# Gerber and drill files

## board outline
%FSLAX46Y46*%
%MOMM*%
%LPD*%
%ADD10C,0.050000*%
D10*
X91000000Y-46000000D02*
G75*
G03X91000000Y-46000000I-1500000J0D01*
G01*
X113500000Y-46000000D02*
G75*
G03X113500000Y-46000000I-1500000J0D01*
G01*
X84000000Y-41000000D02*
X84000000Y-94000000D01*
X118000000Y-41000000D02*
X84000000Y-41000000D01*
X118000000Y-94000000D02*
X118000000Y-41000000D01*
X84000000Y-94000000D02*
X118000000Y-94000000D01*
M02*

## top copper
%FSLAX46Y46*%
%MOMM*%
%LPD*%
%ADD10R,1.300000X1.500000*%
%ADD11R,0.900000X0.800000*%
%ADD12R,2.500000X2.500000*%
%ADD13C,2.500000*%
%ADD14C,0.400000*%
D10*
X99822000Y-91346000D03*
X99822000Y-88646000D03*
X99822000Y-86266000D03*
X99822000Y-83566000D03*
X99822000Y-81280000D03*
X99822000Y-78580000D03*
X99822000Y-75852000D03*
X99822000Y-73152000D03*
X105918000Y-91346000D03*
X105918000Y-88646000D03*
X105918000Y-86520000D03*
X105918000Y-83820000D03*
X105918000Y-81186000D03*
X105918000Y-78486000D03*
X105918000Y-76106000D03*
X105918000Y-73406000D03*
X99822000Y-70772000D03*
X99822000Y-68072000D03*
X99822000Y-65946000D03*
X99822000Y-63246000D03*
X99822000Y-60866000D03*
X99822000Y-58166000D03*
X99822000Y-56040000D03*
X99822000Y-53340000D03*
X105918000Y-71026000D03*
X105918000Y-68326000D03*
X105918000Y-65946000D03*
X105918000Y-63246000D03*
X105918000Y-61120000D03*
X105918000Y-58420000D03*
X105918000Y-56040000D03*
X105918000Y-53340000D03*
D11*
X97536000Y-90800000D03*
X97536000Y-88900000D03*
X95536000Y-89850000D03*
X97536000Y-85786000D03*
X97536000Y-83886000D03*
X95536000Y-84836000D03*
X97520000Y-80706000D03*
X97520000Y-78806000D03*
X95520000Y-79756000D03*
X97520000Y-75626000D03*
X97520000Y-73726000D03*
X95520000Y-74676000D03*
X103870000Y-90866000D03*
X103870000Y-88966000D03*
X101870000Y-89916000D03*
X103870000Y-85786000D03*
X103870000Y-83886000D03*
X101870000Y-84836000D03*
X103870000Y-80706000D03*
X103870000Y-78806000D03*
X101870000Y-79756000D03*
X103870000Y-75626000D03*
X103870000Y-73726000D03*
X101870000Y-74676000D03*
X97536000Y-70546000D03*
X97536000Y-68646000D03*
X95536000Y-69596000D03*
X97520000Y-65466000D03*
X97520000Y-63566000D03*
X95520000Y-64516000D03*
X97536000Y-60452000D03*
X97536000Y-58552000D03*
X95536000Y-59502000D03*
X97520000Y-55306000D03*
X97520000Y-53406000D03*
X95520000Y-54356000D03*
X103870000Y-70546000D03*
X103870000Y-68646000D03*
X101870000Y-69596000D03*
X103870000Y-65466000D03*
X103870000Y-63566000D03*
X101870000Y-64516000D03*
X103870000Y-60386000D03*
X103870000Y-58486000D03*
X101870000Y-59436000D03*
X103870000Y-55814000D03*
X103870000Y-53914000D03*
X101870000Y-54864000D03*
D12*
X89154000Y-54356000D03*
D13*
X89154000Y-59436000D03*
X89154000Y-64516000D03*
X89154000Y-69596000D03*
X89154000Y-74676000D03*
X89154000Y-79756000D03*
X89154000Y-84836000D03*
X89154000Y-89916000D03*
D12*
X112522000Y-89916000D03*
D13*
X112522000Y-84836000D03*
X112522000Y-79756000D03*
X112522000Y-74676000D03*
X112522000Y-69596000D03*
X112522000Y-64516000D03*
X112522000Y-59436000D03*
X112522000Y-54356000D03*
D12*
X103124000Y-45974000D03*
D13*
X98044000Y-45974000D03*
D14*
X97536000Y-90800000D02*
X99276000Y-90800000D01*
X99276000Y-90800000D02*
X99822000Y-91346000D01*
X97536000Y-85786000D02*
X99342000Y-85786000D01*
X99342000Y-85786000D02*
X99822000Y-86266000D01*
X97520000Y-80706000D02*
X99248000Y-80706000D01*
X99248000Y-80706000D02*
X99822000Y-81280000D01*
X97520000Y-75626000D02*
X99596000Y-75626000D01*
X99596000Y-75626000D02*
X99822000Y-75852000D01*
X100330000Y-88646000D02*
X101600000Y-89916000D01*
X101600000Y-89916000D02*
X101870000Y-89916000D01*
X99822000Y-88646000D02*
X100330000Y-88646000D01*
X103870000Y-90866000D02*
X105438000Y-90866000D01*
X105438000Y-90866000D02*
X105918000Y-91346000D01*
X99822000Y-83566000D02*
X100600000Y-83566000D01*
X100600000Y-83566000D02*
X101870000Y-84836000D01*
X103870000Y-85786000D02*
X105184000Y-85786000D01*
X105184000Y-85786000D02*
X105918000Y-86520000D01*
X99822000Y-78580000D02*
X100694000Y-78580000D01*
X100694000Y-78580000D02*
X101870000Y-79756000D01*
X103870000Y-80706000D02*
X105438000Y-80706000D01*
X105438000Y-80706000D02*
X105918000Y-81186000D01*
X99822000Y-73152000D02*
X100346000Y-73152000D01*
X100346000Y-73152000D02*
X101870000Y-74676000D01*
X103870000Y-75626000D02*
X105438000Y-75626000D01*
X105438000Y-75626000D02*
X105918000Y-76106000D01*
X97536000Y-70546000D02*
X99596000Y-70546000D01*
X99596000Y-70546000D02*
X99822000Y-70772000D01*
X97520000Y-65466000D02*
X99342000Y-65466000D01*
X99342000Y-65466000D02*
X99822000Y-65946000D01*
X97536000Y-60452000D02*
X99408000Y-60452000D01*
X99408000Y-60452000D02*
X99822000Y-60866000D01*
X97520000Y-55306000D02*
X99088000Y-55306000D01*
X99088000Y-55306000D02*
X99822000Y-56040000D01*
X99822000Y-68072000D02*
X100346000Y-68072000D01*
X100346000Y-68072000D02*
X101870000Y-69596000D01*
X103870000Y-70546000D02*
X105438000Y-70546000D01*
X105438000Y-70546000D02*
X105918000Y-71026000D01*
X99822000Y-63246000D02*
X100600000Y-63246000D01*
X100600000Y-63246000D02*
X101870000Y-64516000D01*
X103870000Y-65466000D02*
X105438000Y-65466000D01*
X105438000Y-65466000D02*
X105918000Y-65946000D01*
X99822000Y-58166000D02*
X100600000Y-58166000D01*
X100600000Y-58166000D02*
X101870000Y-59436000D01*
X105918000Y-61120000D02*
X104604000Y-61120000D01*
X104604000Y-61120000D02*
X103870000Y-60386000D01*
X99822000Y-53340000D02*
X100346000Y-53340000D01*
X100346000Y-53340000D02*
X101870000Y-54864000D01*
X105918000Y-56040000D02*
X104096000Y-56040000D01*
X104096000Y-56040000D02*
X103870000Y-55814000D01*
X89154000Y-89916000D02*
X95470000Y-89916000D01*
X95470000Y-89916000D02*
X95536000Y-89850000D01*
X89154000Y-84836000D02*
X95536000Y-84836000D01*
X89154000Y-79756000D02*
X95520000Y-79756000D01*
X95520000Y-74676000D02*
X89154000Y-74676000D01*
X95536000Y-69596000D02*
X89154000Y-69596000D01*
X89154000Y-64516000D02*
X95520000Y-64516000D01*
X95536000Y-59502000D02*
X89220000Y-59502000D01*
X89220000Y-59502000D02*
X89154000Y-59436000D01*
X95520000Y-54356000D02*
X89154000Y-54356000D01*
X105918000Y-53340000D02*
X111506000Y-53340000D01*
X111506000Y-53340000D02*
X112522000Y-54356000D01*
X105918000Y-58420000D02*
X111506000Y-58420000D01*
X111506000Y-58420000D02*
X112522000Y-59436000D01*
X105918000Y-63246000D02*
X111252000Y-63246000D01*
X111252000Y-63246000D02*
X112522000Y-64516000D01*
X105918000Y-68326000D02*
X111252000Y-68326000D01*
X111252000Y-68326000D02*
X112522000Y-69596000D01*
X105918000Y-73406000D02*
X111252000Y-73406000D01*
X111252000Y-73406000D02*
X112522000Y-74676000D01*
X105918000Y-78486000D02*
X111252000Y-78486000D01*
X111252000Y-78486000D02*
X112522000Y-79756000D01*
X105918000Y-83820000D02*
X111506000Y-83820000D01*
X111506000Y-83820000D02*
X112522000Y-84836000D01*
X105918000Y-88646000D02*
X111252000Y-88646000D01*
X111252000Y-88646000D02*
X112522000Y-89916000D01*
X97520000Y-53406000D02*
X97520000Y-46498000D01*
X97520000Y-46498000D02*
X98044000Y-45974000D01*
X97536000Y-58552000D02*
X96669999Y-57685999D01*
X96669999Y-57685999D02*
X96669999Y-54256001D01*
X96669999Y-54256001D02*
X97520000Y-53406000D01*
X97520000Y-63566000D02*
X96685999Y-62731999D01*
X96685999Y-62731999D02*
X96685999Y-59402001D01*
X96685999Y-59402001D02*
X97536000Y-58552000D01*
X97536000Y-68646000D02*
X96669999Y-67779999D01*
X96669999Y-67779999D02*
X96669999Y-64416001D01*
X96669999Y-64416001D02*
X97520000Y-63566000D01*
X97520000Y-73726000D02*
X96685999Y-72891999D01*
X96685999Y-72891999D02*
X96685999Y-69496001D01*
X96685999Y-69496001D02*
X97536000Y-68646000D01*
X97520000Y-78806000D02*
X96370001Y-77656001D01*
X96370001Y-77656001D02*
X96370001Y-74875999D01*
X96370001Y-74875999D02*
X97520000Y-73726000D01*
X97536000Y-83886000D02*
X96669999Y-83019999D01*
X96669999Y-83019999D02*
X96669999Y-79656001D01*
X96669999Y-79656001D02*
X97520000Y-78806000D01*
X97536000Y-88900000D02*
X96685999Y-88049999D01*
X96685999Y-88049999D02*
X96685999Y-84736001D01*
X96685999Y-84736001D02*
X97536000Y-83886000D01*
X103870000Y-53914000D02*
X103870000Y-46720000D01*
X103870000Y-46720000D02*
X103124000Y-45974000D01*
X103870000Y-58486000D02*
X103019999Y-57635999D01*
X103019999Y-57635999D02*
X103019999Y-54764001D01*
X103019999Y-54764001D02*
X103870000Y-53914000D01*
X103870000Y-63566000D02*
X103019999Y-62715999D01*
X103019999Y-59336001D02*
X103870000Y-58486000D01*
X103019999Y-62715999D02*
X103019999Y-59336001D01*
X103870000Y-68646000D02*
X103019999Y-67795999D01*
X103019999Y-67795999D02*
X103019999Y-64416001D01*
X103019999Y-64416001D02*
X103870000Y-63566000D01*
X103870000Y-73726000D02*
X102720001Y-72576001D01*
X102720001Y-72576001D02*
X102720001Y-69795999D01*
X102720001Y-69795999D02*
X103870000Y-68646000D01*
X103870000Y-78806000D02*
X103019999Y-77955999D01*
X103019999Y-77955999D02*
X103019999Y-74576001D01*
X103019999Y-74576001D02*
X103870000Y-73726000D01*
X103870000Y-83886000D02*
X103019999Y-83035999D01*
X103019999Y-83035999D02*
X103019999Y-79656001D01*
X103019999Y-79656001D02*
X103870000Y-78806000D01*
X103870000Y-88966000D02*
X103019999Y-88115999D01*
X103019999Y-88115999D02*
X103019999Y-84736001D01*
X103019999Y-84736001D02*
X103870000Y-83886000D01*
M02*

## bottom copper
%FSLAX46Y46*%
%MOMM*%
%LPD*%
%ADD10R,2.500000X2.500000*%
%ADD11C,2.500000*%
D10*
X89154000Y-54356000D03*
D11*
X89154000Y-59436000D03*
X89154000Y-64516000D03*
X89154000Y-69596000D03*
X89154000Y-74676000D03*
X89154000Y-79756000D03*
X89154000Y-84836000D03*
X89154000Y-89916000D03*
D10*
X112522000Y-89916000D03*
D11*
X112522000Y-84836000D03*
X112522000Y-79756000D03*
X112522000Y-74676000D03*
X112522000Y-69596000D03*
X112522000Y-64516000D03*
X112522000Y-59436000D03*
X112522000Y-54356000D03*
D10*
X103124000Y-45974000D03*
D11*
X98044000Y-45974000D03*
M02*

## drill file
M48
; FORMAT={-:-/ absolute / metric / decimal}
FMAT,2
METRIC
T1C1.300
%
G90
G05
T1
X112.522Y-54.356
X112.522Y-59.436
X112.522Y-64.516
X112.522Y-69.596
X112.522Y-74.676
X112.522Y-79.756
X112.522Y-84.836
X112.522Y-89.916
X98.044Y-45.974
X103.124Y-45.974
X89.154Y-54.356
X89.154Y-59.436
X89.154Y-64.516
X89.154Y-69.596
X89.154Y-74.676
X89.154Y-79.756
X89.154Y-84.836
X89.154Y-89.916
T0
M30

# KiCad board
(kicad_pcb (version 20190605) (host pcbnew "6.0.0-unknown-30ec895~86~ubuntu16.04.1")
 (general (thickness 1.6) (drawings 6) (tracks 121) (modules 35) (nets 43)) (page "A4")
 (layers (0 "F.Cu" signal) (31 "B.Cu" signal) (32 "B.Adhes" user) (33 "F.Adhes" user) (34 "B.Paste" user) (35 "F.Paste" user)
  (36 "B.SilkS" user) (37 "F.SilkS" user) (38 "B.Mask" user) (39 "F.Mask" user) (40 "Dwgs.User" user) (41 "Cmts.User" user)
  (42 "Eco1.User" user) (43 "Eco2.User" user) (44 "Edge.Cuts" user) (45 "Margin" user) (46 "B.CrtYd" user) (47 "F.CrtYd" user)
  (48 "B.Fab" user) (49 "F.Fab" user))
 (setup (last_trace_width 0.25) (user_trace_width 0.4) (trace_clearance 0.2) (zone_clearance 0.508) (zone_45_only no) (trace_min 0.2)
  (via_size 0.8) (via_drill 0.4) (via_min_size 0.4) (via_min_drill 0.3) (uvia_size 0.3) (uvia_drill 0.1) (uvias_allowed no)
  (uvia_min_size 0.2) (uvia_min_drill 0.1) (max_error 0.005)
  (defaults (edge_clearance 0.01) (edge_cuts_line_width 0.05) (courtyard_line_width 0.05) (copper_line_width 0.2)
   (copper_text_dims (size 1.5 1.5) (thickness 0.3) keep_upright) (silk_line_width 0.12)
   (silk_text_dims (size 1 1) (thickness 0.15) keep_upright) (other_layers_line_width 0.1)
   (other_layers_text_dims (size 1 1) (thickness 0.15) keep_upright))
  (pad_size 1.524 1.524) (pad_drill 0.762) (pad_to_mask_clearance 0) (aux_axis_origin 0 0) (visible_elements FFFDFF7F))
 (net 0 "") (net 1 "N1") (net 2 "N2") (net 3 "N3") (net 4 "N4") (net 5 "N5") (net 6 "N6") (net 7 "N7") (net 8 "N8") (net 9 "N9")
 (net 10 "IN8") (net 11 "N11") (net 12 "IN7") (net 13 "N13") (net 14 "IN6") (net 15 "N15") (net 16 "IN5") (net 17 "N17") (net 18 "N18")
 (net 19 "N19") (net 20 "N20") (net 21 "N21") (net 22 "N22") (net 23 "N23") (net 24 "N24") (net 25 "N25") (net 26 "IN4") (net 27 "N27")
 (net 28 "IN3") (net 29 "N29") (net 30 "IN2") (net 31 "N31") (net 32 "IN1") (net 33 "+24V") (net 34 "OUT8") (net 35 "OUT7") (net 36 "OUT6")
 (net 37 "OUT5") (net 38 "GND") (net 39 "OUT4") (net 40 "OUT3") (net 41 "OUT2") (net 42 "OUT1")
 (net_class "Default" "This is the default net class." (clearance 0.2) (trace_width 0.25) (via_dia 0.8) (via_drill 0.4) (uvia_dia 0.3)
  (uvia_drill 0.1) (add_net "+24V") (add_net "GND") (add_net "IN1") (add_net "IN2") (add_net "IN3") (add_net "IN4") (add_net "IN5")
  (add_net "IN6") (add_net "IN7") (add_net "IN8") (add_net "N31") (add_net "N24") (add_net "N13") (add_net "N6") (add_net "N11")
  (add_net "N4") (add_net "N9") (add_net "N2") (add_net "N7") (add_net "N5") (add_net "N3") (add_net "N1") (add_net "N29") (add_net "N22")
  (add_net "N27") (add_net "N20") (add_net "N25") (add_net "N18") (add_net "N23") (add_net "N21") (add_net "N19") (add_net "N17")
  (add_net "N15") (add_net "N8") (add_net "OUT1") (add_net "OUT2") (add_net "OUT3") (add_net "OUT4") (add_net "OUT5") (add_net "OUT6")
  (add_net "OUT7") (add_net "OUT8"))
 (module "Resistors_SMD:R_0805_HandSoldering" (layer "F.Cu") (at 99.822 89.996 90)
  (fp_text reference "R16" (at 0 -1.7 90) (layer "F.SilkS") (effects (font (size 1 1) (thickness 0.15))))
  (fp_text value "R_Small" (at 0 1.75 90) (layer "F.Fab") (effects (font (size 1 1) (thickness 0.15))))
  (pad "1" smd rect (at -1.35 0 90) (size 1.5 1.3) (layers "F.Cu" "F.Paste" "F.Mask") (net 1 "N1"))
  (pad "2" smd rect (at 1.35 0 90) (size 1.5 1.3) (layers "F.Cu" "F.Paste" "F.Mask") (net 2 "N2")))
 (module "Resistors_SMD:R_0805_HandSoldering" (layer "F.Cu") (at 99.822 84.916 90)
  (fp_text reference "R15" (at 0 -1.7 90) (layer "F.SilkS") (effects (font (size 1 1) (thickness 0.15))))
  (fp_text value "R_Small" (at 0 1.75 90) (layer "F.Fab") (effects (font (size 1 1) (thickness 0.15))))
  (pad "1" smd rect (at -1.35 0 90) (size 1.5 1.3) (layers "F.Cu" "F.Paste" "F.Mask") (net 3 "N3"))
  (pad "2" smd rect (at 1.35 0 90) (size 1.5 1.3) (layers "F.Cu" "F.Paste" "F.Mask") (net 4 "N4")))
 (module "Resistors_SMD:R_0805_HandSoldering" (layer "F.Cu") (at 99.822 79.93 90)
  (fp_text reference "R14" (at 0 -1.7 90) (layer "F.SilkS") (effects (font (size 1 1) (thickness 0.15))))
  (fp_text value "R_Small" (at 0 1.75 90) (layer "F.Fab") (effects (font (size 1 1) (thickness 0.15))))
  (pad "1" smd rect (at -1.35 0 90) (size 1.5 1.3) (layers "F.Cu" "F.Paste" "F.Mask") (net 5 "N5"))
  (pad "2" smd rect (at 1.35 0 90) (size 1.5 1.3) (layers "F.Cu" "F.Paste" "F.Mask") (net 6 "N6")))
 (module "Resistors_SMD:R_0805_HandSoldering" (layer "F.Cu") (at 99.822 74.502 90)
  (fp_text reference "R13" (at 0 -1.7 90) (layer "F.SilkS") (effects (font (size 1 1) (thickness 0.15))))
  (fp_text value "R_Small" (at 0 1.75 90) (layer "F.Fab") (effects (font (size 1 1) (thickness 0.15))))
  (pad "1" smd rect (at -1.35 0 90) (size 1.5 1.3) (layers "F.Cu" "F.Paste" "F.Mask") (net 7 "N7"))
  (pad "2" smd rect (at 1.35 0 90) (size 1.5 1.3) (layers "F.Cu" "F.Paste" "F.Mask") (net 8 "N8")))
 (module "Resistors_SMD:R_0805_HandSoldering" (layer "F.Cu") (at 105.918 89.996 90)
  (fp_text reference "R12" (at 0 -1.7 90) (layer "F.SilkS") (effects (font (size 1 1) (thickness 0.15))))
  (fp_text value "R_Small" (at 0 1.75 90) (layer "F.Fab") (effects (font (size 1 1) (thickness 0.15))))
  (pad "1" smd rect (at -1.35 0 90) (size 1.5 1.3) (layers "F.Cu" "F.Paste" "F.Mask") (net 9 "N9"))
  (pad "2" smd rect (at 1.35 0 90) (size 1.5 1.3) (layers "F.Cu" "F.Paste" "F.Mask") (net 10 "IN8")))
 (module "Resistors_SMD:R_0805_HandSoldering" (layer "F.Cu") (at 105.918 85.17 90)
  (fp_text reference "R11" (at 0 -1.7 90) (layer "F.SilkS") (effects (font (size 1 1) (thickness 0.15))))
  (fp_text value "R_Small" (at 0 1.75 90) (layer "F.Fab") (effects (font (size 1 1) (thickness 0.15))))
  (pad "1" smd rect (at -1.35 0 90) (size 1.5 1.3) (layers "F.Cu" "F.Paste" "F.Mask") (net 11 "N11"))
  (pad "2" smd rect (at 1.35 0 90) (size 1.5 1.3) (layers "F.Cu" "F.Paste" "F.Mask") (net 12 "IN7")))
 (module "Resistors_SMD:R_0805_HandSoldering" (layer "F.Cu") (at 105.918 79.836 90)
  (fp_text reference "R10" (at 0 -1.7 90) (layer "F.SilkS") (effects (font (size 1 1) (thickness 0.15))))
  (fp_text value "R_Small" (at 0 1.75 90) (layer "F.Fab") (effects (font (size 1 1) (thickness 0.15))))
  (pad "1" smd rect (at -1.35 0 90) (size 1.5 1.3) (layers "F.Cu" "F.Paste" "F.Mask") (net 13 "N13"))
  (pad "2" smd rect (at 1.35 0 90) (size 1.5 1.3) (layers "F.Cu" "F.Paste" "F.Mask") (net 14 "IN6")))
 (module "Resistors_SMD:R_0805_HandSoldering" (layer "F.Cu") (at 105.918 74.756 90)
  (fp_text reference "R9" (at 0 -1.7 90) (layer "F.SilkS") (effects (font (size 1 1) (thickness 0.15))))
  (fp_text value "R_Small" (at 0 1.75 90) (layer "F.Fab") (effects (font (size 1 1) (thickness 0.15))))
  (pad "1" smd rect (at -1.35 0 90) (size 1.5 1.3) (layers "F.Cu" "F.Paste" "F.Mask") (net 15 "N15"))
  (pad "2" smd rect (at 1.35 0 90) (size 1.5 1.3) (layers "F.Cu" "F.Paste" "F.Mask") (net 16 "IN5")))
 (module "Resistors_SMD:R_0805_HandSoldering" (layer "F.Cu") (at 99.822 69.422 90)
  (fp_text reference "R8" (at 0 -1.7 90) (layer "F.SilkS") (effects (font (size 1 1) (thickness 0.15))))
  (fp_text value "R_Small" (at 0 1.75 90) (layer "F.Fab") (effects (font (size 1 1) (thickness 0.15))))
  (pad "1" smd rect (at -1.35 0 90) (size 1.5 1.3) (layers "F.Cu" "F.Paste" "F.Mask") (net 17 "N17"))
  (pad "2" smd rect (at 1.35 0 90) (size 1.5 1.3) (layers "F.Cu" "F.Paste" "F.Mask") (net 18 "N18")))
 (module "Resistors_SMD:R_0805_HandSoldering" (layer "F.Cu") (at 99.822 64.596 90)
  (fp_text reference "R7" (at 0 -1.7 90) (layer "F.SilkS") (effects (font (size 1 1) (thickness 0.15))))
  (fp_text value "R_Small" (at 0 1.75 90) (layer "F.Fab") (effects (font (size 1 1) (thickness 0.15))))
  (pad "1" smd rect (at -1.35 0 90) (size 1.5 1.3) (layers "F.Cu" "F.Paste" "F.Mask") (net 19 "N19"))
  (pad "2" smd rect (at 1.35 0 90) (size 1.5 1.3) (layers "F.Cu" "F.Paste" "F.Mask") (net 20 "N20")))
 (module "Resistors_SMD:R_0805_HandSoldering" (layer "F.Cu") (at 99.822 59.516 90)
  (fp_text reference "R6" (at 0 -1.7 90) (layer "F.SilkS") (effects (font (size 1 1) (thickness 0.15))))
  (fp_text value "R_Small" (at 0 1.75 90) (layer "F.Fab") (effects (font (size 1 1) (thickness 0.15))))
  (pad "1" smd rect (at -1.35 0 90) (size 1.5 1.3) (layers "F.Cu" "F.Paste" "F.Mask") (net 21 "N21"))
  (pad "2" smd rect (at 1.35 0 90) (size 1.5 1.3) (layers "F.Cu" "F.Paste" "F.Mask") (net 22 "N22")))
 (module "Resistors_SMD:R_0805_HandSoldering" (layer "F.Cu") (at 99.822 54.69 90)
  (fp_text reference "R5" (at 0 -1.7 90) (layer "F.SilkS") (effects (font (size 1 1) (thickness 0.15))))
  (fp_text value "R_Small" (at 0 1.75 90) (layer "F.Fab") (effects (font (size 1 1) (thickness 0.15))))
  (pad "1" smd rect (at -1.35 0 90) (size 1.5 1.3) (layers "F.Cu" "F.Paste" "F.Mask") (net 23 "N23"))
  (pad "2" smd rect (at 1.35 0 90) (size 1.5 1.3) (layers "F.Cu" "F.Paste" "F.Mask") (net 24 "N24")))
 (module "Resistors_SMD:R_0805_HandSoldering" (layer "F.Cu") (at 105.918 69.676 90)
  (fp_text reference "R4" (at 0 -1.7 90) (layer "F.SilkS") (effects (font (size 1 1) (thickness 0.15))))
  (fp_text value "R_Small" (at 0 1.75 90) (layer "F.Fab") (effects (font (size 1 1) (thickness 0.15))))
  (pad "1" smd rect (at -1.35 0 90) (size 1.5 1.3) (layers "F.Cu" "F.Paste" "F.Mask") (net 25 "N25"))
  (pad "2" smd rect (at 1.35 0 90) (size 1.5 1.3) (layers "F.Cu" "F.Paste" "F.Mask") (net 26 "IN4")))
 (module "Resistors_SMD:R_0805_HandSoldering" (layer "F.Cu") (at 105.918 64.596 90)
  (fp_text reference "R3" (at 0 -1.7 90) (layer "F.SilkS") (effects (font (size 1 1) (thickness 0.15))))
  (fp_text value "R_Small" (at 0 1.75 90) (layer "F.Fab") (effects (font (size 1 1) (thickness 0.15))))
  (pad "1" smd rect (at -1.35 0 90) (size 1.5 1.3) (layers "F.Cu" "F.Paste" "F.Mask") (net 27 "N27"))
  (pad "2" smd rect (at 1.35 0 90) (size 1.5 1.3) (layers "F.Cu" "F.Paste" "F.Mask") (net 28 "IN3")))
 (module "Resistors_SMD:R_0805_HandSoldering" (layer "F.Cu") (at 105.918 59.77 90)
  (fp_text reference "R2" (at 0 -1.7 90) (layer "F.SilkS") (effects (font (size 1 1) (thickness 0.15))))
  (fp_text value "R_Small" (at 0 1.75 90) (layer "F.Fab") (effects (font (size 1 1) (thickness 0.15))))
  (pad "1" smd rect (at -1.35 0 90) (size 1.5 1.3) (layers "F.Cu" "F.Paste" "F.Mask") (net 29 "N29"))
  (pad "2" smd rect (at 1.35 0 90) (size 1.5 1.3) (layers "F.Cu" "F.Paste" "F.Mask") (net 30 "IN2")))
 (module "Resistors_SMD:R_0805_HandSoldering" (layer "F.Cu") (at 105.918 54.69 90)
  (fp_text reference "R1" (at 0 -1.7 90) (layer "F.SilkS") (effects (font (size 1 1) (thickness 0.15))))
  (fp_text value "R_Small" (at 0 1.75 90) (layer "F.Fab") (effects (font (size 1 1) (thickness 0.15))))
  (pad "1" smd rect (at -1.35 0 90) (size 1.5 1.3) (layers "F.Cu" "F.Paste" "F.Mask") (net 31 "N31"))
  (pad "2" smd rect (at 1.35 0 90) (size 1.5 1.3) (layers "F.Cu" "F.Paste" "F.Mask") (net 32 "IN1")))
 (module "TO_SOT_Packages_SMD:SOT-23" (layer "F.Cu") (at 96.536 89.85 180)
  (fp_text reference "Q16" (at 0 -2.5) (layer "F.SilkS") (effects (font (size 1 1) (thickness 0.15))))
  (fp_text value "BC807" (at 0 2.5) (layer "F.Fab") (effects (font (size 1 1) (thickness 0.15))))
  (pad "1" smd rect (at -1 -0.95 180) (size 0.9 0.8) (layers "F.Cu" "F.Paste" "F.Mask") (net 1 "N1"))
  (pad "2" smd rect (at -1 0.95 180) (size 0.9 0.8) (layers "F.Cu" "F.Paste" "F.Mask") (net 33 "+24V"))
  (pad "3" smd rect (at 1 0 180) (size 0.9 0.8) (layers "F.Cu" "F.Paste" "F.Mask") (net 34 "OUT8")))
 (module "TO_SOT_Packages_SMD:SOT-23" (layer "F.Cu") (at 96.536 84.836 180)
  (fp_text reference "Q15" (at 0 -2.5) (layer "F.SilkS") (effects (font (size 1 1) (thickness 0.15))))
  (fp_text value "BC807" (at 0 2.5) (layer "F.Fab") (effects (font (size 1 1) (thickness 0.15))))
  (pad "1" smd rect (at -1 -0.95 180) (size 0.9 0.8) (layers "F.Cu" "F.Paste" "F.Mask") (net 3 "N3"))
  (pad "2" smd rect (at -1 0.95 180) (size 0.9 0.8) (layers "F.Cu" "F.Paste" "F.Mask") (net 33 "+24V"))
  (pad "3" smd rect (at 1 0 180) (size 0.9 0.8) (layers "F.Cu" "F.Paste" "F.Mask") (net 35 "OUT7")))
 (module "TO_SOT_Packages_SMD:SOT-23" (layer "F.Cu") (at 96.52 79.756 180)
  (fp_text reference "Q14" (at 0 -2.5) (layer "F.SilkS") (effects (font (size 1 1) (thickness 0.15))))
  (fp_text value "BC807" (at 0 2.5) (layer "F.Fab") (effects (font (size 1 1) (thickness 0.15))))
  (pad "1" smd rect (at -1 -0.95 180) (size 0.9 0.8) (layers "F.Cu" "F.Paste" "F.Mask") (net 5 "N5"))
  (pad "2" smd rect (at -1 0.95 180) (size 0.9 0.8) (layers "F.Cu" "F.Paste" "F.Mask") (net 33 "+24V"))
  (pad "3" smd rect (at 1 0 180) (size 0.9 0.8) (layers "F.Cu" "F.Paste" "F.Mask") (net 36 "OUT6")))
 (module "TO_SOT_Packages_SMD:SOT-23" (layer "F.Cu") (at 96.52 74.676 180)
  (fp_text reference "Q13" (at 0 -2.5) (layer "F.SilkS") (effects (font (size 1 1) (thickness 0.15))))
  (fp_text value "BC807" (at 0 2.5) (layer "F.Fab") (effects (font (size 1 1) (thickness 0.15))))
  (pad "1" smd rect (at -1 -0.95 180) (size 0.9 0.8) (layers "F.Cu" "F.Paste" "F.Mask") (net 7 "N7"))
  (pad "2" smd rect (at -1 0.95 180) (size 0.9 0.8) (layers "F.Cu" "F.Paste" "F.Mask") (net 33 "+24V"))
  (pad "3" smd rect (at 1 0 180) (size 0.9 0.8) (layers "F.Cu" "F.Paste" "F.Mask") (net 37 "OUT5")))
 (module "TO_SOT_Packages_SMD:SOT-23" (layer "F.Cu") (at 102.87 89.916 180)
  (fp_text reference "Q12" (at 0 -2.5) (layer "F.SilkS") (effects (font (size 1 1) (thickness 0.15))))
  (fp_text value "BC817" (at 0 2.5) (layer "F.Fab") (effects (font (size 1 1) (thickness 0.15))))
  (pad "1" smd rect (at -1 -0.95 180) (size 0.9 0.8) (layers "F.Cu" "F.Paste" "F.Mask") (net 9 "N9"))
  (pad "2" smd rect (at -1 0.95 180) (size 0.9 0.8) (layers "F.Cu" "F.Paste" "F.Mask") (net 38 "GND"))
  (pad "3" smd rect (at 1 0 180) (size 0.9 0.8) (layers "F.Cu" "F.Paste" "F.Mask") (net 2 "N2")))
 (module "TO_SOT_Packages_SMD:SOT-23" (layer "F.Cu") (at 102.87 84.836 180)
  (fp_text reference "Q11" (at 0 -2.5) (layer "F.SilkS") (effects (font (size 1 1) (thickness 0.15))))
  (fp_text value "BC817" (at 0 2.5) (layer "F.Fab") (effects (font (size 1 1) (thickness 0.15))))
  (pad "1" smd rect (at -1 -0.95 180) (size 0.9 0.8) (layers "F.Cu" "F.Paste" "F.Mask") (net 11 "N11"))
  (pad "2" smd rect (at -1 0.95 180) (size 0.9 0.8) (layers "F.Cu" "F.Paste" "F.Mask") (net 38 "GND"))
  (pad "3" smd rect (at 1 0 180) (size 0.9 0.8) (layers "F.Cu" "F.Paste" "F.Mask") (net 4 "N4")))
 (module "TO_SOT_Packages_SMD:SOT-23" (layer "F.Cu") (at 102.87 79.756 180)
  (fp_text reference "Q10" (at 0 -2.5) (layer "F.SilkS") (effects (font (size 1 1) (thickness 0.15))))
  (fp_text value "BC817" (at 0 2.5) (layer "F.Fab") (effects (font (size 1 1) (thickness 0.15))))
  (pad "1" smd rect (at -1 -0.95 180) (size 0.9 0.8) (layers "F.Cu" "F.Paste" "F.Mask") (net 13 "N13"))
  (pad "2" smd rect (at -1 0.95 180) (size 0.9 0.8) (layers "F.Cu" "F.Paste" "F.Mask") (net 38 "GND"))
  (pad "3" smd rect (at 1 0 180) (size 0.9 0.8) (layers "F.Cu" "F.Paste" "F.Mask") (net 6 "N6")))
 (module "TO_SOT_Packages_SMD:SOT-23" (layer "F.Cu") (at 102.87 74.676 180)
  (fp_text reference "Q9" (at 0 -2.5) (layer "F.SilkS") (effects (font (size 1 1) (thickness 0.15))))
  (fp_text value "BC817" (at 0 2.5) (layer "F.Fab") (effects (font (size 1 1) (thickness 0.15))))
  (pad "1" smd rect (at -1 -0.95 180) (size 0.9 0.8) (layers "F.Cu" "F.Paste" "F.Mask") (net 15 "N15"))
  (pad "2" smd rect (at -1 0.95 180) (size 0.9 0.8) (layers "F.Cu" "F.Paste" "F.Mask") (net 38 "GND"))
  (pad "3" smd rect (at 1 0 180) (size 0.9 0.8) (layers "F.Cu" "F.Paste" "F.Mask") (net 8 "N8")))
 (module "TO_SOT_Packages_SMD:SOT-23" (layer "F.Cu") (at 96.536 69.596 180)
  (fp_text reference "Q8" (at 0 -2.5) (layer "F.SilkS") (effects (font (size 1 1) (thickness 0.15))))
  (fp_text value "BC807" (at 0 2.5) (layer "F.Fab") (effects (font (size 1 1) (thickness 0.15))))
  (pad "1" smd rect (at -1 -0.95 180) (size 0.9 0.8) (layers "F.Cu" "F.Paste" "F.Mask") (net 17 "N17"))
  (pad "2" smd rect (at -1 0.95 180) (size 0.9 0.8) (layers "F.Cu" "F.Paste" "F.Mask") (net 33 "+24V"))
  (pad "3" smd rect (at 1 0 180) (size 0.9 0.8) (layers "F.Cu" "F.Paste" "F.Mask") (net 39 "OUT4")))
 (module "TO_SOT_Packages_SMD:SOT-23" (layer "F.Cu") (at 96.52 64.516 180)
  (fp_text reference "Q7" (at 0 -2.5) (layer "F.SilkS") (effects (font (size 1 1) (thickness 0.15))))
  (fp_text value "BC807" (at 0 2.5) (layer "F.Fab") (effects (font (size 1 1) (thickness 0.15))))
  (pad "1" smd rect (at -1 -0.95 180) (size 0.9 0.8) (layers "F.Cu" "F.Paste" "F.Mask") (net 19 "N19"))
  (pad "2" smd rect (at -1 0.95 180) (size 0.9 0.8) (layers "F.Cu" "F.Paste" "F.Mask") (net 33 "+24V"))
  (pad "3" smd rect (at 1 0 180) (size 0.9 0.8) (layers "F.Cu" "F.Paste" "F.Mask") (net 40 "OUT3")))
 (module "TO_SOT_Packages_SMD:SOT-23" (layer "F.Cu") (at 96.536 59.502 180)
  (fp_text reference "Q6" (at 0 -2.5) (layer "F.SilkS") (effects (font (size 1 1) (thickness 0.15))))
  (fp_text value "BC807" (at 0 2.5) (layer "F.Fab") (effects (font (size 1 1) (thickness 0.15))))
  (pad "1" smd rect (at -1 -0.95 180) (size 0.9 0.8) (layers "F.Cu" "F.Paste" "F.Mask") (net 21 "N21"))
  (pad "2" smd rect (at -1 0.95 180) (size 0.9 0.8) (layers "F.Cu" "F.Paste" "F.Mask") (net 33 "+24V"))
  (pad "3" smd rect (at 1 0 180) (size 0.9 0.8) (layers "F.Cu" "F.Paste" "F.Mask") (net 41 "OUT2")))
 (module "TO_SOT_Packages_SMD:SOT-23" (layer "F.Cu") (at 96.52 54.356 180)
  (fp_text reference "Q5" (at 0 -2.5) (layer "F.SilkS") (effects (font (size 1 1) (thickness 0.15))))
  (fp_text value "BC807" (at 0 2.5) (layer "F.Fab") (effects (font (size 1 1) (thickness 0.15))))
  (pad "1" smd rect (at -1 -0.95 180) (size 0.9 0.8) (layers "F.Cu" "F.Paste" "F.Mask") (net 23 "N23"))
  (pad "2" smd rect (at -1 0.95 180) (size 0.9 0.8) (layers "F.Cu" "F.Paste" "F.Mask") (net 33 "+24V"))
  (pad "3" smd rect (at 1 0 180) (size 0.9 0.8) (layers "F.Cu" "F.Paste" "F.Mask") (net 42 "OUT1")))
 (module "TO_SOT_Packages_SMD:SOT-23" (layer "F.Cu") (at 102.87 69.596 180)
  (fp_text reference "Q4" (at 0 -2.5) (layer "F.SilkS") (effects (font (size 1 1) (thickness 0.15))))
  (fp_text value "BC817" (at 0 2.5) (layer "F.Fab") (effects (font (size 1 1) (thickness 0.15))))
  (pad "1" smd rect (at -1 -0.95 180) (size 0.9 0.8) (layers "F.Cu" "F.Paste" "F.Mask") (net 25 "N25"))
  (pad "2" smd rect (at -1 0.95 180) (size 0.9 0.8) (layers "F.Cu" "F.Paste" "F.Mask") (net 38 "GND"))
  (pad "3" smd rect (at 1 0 180) (size 0.9 0.8) (layers "F.Cu" "F.Paste" "F.Mask") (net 18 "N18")))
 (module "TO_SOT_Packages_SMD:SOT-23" (layer "F.Cu") (at 102.87 64.516 180)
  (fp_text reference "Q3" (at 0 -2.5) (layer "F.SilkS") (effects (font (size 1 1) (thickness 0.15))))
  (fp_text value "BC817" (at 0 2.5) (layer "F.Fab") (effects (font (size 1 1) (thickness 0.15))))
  (pad "1" smd rect (at -1 -0.95 180) (size 0.9 0.8) (layers "F.Cu" "F.Paste" "F.Mask") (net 27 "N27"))
  (pad "2" smd rect (at -1 0.95 180) (size 0.9 0.8) (layers "F.Cu" "F.Paste" "F.Mask") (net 38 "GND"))
  (pad "3" smd rect (at 1 0 180) (size 0.9 0.8) (layers "F.Cu" "F.Paste" "F.Mask") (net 20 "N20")))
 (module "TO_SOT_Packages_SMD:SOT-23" (layer "F.Cu") (at 102.87 59.436 180)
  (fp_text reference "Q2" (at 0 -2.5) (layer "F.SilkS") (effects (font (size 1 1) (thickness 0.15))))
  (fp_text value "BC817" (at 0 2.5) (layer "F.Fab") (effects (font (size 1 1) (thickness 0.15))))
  (pad "1" smd rect (at -1 -0.95 180) (size 0.9 0.8) (layers "F.Cu" "F.Paste" "F.Mask") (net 29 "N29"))
  (pad "2" smd rect (at -1 0.95 180) (size 0.9 0.8) (layers "F.Cu" "F.Paste" "F.Mask") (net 38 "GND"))
  (pad "3" smd rect (at 1 0 180) (size 0.9 0.8) (layers "F.Cu" "F.Paste" "F.Mask") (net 22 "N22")))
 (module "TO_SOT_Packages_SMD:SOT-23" (layer "F.Cu") (at 102.87 54.864 180)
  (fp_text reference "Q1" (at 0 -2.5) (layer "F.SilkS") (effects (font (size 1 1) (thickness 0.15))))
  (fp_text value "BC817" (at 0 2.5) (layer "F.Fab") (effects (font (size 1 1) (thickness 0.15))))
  (pad "1" smd rect (at -1 -0.95 180) (size 0.9 0.8) (layers "F.Cu" "F.Paste" "F.Mask") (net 31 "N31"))
  (pad "2" smd rect (at -1 0.95 180) (size 0.9 0.8) (layers "F.Cu" "F.Paste" "F.Mask") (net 38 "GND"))
  (pad "3" smd rect (at 1 0 180) (size 0.9 0.8) (layers "F.Cu" "F.Paste" "F.Mask") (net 24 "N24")))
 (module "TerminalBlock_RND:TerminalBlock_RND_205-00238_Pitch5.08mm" (layer "F.Cu") (at 89.154 54.356 270)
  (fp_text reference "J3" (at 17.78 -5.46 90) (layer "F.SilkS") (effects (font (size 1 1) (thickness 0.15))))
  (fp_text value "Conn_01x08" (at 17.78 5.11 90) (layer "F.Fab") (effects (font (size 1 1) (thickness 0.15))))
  (pad "1" thru_hole rect (at 0 0 270) (size 2.5 2.5) (drill 1.3) (layers *.Cu *.Mask) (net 42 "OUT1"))
  (pad "2" thru_hole circle (at 5.08 0 270) (size 2.5 2.5) (drill 1.3) (layers *.Cu *.Mask) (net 41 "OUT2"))
  (pad "3" thru_hole circle (at 10.16 0 270) (size 2.5 2.5) (drill 1.3) (layers *.Cu *.Mask) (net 40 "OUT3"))
  (pad "4" thru_hole circle (at 15.24 0 270) (size 2.5 2.5) (drill 1.3) (layers *.Cu *.Mask) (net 39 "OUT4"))
  (pad "5" thru_hole circle (at 20.32 0 270) (size 2.5 2.5) (drill 1.3) (layers *.Cu *.Mask) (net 37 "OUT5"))
  (pad "6" thru_hole circle (at 25.4 0 270) (size 2.5 2.5) (drill 1.3) (layers *.Cu *.Mask) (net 36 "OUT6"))
  (pad "7" thru_hole circle (at 30.48 0 270) (size 2.5 2.5) (drill 1.3) (layers *.Cu *.Mask) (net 35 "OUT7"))
  (pad "8" thru_hole circle (at 35.56 0 270) (size 2.5 2.5) (drill 1.3) (layers *.Cu *.Mask) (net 34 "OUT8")))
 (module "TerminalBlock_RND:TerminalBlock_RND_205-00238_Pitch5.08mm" (layer "F.Cu") (at 112.522 89.916 90)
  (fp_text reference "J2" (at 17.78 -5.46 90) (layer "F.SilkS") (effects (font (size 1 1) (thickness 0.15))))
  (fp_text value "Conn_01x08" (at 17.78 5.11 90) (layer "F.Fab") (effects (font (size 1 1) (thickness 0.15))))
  (pad "1" thru_hole rect (at 0 0 90) (size 2.5 2.5) (drill 1.3) (layers *.Cu *.Mask) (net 10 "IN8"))
  (pad "2" thru_hole circle (at 5.08 0 90) (size 2.5 2.5) (drill 1.3) (layers *.Cu *.Mask) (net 12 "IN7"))
  (pad "3" thru_hole circle (at 10.16 0 90) (size 2.5 2.5) (drill 1.3) (layers *.Cu *.Mask) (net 14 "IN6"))
  (pad "4" thru_hole circle (at 15.24 0 90) (size 2.5 2.5) (drill 1.3) (layers *.Cu *.Mask) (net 16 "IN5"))
  (pad "5" thru_hole circle (at 20.32 0 90) (size 2.5 2.5) (drill 1.3) (layers *.Cu *.Mask) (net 26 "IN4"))
  (pad "6" thru_hole circle (at 25.4 0 90) (size 2.5 2.5) (drill 1.3) (layers *.Cu *.Mask) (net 28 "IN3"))
  (pad "7" thru_hole circle (at 30.48 0 90) (size 2.5 2.5) (drill 1.3) (layers *.Cu *.Mask) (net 30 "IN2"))
  (pad "8" thru_hole circle (at 35.56 0 90) (size 2.5 2.5) (drill 1.3) (layers *.Cu *.Mask) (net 32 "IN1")))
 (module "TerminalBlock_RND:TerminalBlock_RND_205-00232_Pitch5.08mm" (layer "F.Cu") (at 103.124 45.974 180)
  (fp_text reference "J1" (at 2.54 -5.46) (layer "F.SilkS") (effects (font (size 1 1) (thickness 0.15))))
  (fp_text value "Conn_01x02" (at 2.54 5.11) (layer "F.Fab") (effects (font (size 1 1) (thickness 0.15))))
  (pad "1" thru_hole rect (at 0 0 180) (size 2.5 2.5) (drill 1.3) (layers *.Cu *.Mask) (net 38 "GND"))
  (pad "2" thru_hole circle (at 5.08 0 180) (size 2.5 2.5) (drill 1.3) (layers *.Cu *.Mask) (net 33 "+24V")))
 (gr_circle (center 89.5 46) (end 91 46) (layer "Edge.Cuts") (width 0.05))
 (gr_circle (center 112 46) (end 113.5 46) (layer "Edge.Cuts") (width 0.05))
 (gr_line (start 84 41) (end 84 94) (layer "Edge.Cuts") (width 0.05))
 (gr_line (start 118 41) (end 84 41) (layer "Edge.Cuts") (width 0.05))
 (gr_line (start 118 94) (end 118 41) (layer "Edge.Cuts") (width 0.05))
 (gr_line (start 84 94) (end 118 94) (layer "Edge.Cuts") (width 0.05))
 (segment (start 97.536 90.8) (end 99.276 90.8) (width 0.4) (layer "F.Cu") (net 1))
 (segment (start 99.276 90.8) (end 99.822 91.346) (width 0.4) (layer "F.Cu") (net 1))
 (segment (start 97.536 85.786) (end 99.342 85.786) (width 0.4) (layer "F.Cu") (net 3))
 (segment (start 99.342 85.786) (end 99.822 86.266) (width 0.4) (layer "F.Cu") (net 3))
 (segment (start 97.52 80.706) (end 99.248 80.706) (width 0.4) (layer "F.Cu") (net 5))
 (segment (start 99.248 80.706) (end 99.822 81.28) (width 0.4) (layer "F.Cu") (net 5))
 (segment (start 97.52 75.626) (end 99.596 75.626) (width 0.4) (layer "F.Cu") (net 7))
 (segment (start 99.596 75.626) (end 99.822 75.852) (width 0.4) (layer "F.Cu") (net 7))
 (segment (start 100.33 88.646) (end 101.6 89.916) (width 0.4) (layer "F.Cu") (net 2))
 (segment (start 101.6 89.916) (end 101.87 89.916) (width 0.4) (layer "F.Cu") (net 2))
 (segment (start 99.822 88.646) (end 100.33 88.646) (width 0.4) (layer "F.Cu") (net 2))
 (segment (start 103.87 90.866) (end 105.438 90.866) (width 0.4) (layer "F.Cu") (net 9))
 (segment (start 105.438 90.866) (end 105.918 91.346) (width 0.4) (layer "F.Cu") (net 9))
 (segment (start 99.822 83.566) (end 100.6 83.566) (width 0.4) (layer "F.Cu") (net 4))
 (segment (start 100.6 83.566) (end 101.87 84.836) (width 0.4) (layer "F.Cu") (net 4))
 (segment (start 103.87 85.786) (end 105.184 85.786) (width 0.4) (layer "F.Cu") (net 11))
 (segment (start 105.184 85.786) (end 105.918 86.52) (width 0.4) (layer "F.Cu") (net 11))
 (segment (start 99.822 78.58) (end 100.694 78.58) (width 0.4) (layer "F.Cu") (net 6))
 (segment (start 100.694 78.58) (end 101.87 79.756) (width 0.4) (layer "F.Cu") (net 6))
 (segment (start 103.87 80.706) (end 105.438 80.706) (width 0.4) (layer "F.Cu") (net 13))
 (segment (start 105.438 80.706) (end 105.918 81.186) (width 0.4) (layer "F.Cu") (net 13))
 (segment (start 99.822 73.152) (end 100.346 73.152) (width 0.4) (layer "F.Cu") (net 8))
 (segment (start 100.346 73.152) (end 101.87 74.676) (width 0.4) (layer "F.Cu") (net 8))
 (segment (start 103.87 75.626) (end 105.438 75.626) (width 0.4) (layer "F.Cu") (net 15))
 (segment (start 105.438 75.626) (end 105.918 76.106) (width 0.4) (layer "F.Cu") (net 15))
 (segment (start 97.536 70.546) (end 99.596 70.546) (width 0.4) (layer "F.Cu") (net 17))
 (segment (start 99.596 70.546) (end 99.822 70.772) (width 0.4) (layer "F.Cu") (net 17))
 (segment (start 97.52 65.466) (end 99.342 65.466) (width 0.4) (layer "F.Cu") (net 19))
 (segment (start 99.342 65.466) (end 99.822 65.946) (width 0.4) (layer "F.Cu") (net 19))
 (segment (start 97.536 60.452) (end 99.408 60.452) (width 0.4) (layer "F.Cu") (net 21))
 (segment (start 99.408 60.452) (end 99.822 60.866) (width 0.4) (layer "F.Cu") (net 21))
 (segment (start 97.52 55.306) (end 99.088 55.306) (width 0.4) (layer "F.Cu") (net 23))
 (segment (start 99.088 55.306) (end 99.822 56.04) (width 0.4) (layer "F.Cu") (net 23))
 (segment (start 99.822 68.072) (end 100.346 68.072) (width 0.4) (layer "F.Cu") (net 18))
 (segment (start 100.346 68.072) (end 101.87 69.596) (width 0.4) (layer "F.Cu") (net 18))
 (segment (start 103.87 70.546) (end 105.438 70.546) (width 0.4) (layer "F.Cu") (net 25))
 (segment (start 105.438 70.546) (end 105.918 71.026) (width 0.4) (layer "F.Cu") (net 25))
 (segment (start 99.822 63.246) (end 100.6 63.246) (width 0.4) (layer "F.Cu") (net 20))
 (segment (start 100.6 63.246) (end 101.87 64.516) (width 0.4) (layer "F.Cu") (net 20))
 (segment (start 103.87 65.466) (end 105.438 65.466) (width 0.4) (layer "F.Cu") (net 27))
 (segment (start 105.438 65.466) (end 105.918 65.946) (width 0.4) (layer "F.Cu") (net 27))
 (segment (start 99.822 58.166) (end 100.6 58.166) (width 0.4) (layer "F.Cu") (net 22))
 (segment (start 100.6 58.166) (end 101.87 59.436) (width 0.4) (layer "F.Cu") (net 22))
 (segment (start 105.918 61.12) (end 104.604 61.12) (width 0.4) (layer "F.Cu") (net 29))
 (segment (start 104.604 61.12) (end 103.87 60.386) (width 0.4) (layer "F.Cu") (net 29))
 (segment (start 99.822 53.34) (end 100.346 53.34) (width 0.4) (layer "F.Cu") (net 24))
 (segment (start 100.346 53.34) (end 101.87 54.864) (width 0.4) (layer "F.Cu") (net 24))
 (segment (start 105.918 56.04) (end 104.096 56.04) (width 0.4) (layer "F.Cu") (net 31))
 (segment (start 104.096 56.04) (end 103.87 55.814) (width 0.4) (layer "F.Cu") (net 31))
 (segment (start 89.154 89.916) (end 95.47 89.916) (width 0.4) (layer "F.Cu") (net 34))
 (segment (start 95.47 89.916) (end 95.536 89.85) (width 0.4) (layer "F.Cu") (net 34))
 (segment (start 89.154 84.836) (end 95.536 84.836) (width 0.4) (layer "F.Cu") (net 35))
 (segment (start 89.154 79.756) (end 95.52 79.756) (width 0.4) (layer "F.Cu") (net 36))
 (segment (start 95.52 74.676) (end 89.154 74.676) (width 0.4) (layer "F.Cu") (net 37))
 (segment (start 95.536 69.596) (end 89.154 69.596) (width 0.4) (layer "F.Cu") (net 39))
 (segment (start 89.154 64.516) (end 95.52 64.516) (width 0.4) (layer "F.Cu") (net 40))
 (segment (start 95.536 59.502) (end 89.22 59.502) (width 0.4) (layer "F.Cu") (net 41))
 (segment (start 89.22 59.502) (end 89.154 59.436) (width 0.4) (layer "F.Cu") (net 41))
 (segment (start 95.52 54.356) (end 89.154 54.356) (width 0.4) (layer "F.Cu") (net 42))
 (segment (start 105.918 53.34) (end 111.506 53.34) (width 0.4) (layer "F.Cu") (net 32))
 (segment (start 111.506 53.34) (end 112.522 54.356) (width 0.4) (layer "F.Cu") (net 32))
 (segment (start 105.918 58.42) (end 111.506 58.42) (width 0.4) (layer "F.Cu") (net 30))
 (segment (start 111.506 58.42) (end 112.522 59.436) (width 0.4) (layer "F.Cu") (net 30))
 (segment (start 105.918 63.246) (end 111.252 63.246) (width 0.4) (layer "F.Cu") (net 28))
 (segment (start 111.252 63.246) (end 112.522 64.516) (width 0.4) (layer "F.Cu") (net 28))
 (segment (start 105.918 68.326) (end 111.252 68.326) (width 0.4) (layer "F.Cu") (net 26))
 (segment (start 111.252 68.326) (end 112.522 69.596) (width 0.4) (layer "F.Cu") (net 26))
 (segment (start 105.918 73.406) (end 111.252 73.406) (width 0.4) (layer "F.Cu") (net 16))
 (segment (start 111.252 73.406) (end 112.522 74.676) (width 0.4) (layer "F.Cu") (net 16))
 (segment (start 105.918 78.486) (end 111.252 78.486) (width 0.4) (layer "F.Cu") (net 14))
 (segment (start 111.252 78.486) (end 112.522 79.756) (width 0.4) (layer "F.Cu") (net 14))
 (segment (start 105.918 83.82) (end 111.506 83.82) (width 0.4) (layer "F.Cu") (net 12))
 (segment (start 111.506 83.82) (end 112.522 84.836) (width 0.4) (layer "F.Cu") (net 12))
 (segment (start 105.918 88.646) (end 111.252 88.646) (width 0.4) (layer "F.Cu") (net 10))
 (segment (start 111.252 88.646) (end 112.522 89.916) (width 0.4) (layer "F.Cu") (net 10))
 (segment (start 97.52 53.406) (end 97.52 46.498) (width 0.4) (layer "F.Cu") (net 33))
 (segment (start 97.52 46.498) (end 98.044 45.974) (width 0.4) (layer "F.Cu") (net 33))
 (segment (start 97.536 58.552) (end 96.669999 57.685999) (width 0.4) (layer "F.Cu") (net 33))
 (segment (start 96.669999 57.685999) (end 96.669999 54.256001) (width 0.4) (layer "F.Cu") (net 33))
 (segment (start 96.669999 54.256001) (end 97.52 53.406) (width 0.4) (layer "F.Cu") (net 33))
 (segment (start 97.52 63.566) (end 96.685999 62.731999) (width 0.4) (layer "F.Cu") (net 33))
 (segment (start 96.685999 62.731999) (end 96.685999 59.402001) (width 0.4) (layer "F.Cu") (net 33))
 (segment (start 96.685999 59.402001) (end 97.536 58.552) (width 0.4) (layer "F.Cu") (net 33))
 (segment (start 97.536 68.646) (end 96.669999 67.779999) (width 0.4) (layer "F.Cu") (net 33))
 (segment (start 96.669999 67.779999) (end 96.669999 64.416001) (width 0.4) (layer "F.Cu") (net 33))
 (segment (start 96.669999 64.416001) (end 97.52 63.566) (width 0.4) (layer "F.Cu") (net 33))
 (segment (start 97.52 73.726) (end 96.685999 72.891999) (width 0.4) (layer "F.Cu") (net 33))
 (segment (start 96.685999 72.891999) (end 96.685999 69.496001) (width 0.4) (layer "F.Cu") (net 33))
 (segment (start 96.685999 69.496001) (end 97.536 68.646) (width 0.4) (layer "F.Cu") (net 33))
 (segment (start 97.52 78.806) (end 96.370001 77.656001) (width 0.4) (layer "F.Cu") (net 33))
 (segment (start 96.370001 77.656001) (end 96.370001 74.875999) (width 0.4) (layer "F.Cu") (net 33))
 (segment (start 96.370001 74.875999) (end 97.52 73.726) (width 0.4) (layer "F.Cu") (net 33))
 (segment (start 97.536 83.886) (end 96.669999 83.019999) (width 0.4) (layer "F.Cu") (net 33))
 (segment (start 96.669999 83.019999) (end 96.669999 79.656001) (width 0.4) (layer "F.Cu") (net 33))
 (segment (start 96.669999 79.656001) (end 97.52 78.806) (width 0.4) (layer "F.Cu") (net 33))
 (segment (start 97.536 88.9) (end 96.685999 88.049999) (width 0.4) (layer "F.Cu") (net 33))
 (segment (start 96.685999 88.049999) (end 96.685999 84.736001) (width 0.4) (layer "F.Cu") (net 33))
 (segment (start 96.685999 84.736001) (end 97.536 83.886) (width 0.4) (layer "F.Cu") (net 33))
 (segment (start 103.87 53.914) (end 103.87 46.72) (width 0.4) (layer "F.Cu") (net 38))
 (segment (start 103.87 46.72) (end 103.124 45.974) (width 0.4) (layer "F.Cu") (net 38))
 (segment (start 103.87 58.486) (end 103.019999 57.635999) (width 0.4) (layer "F.Cu") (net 38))
 (segment (start 103.019999 57.635999) (end 103.019999 54.764001) (width 0.4) (layer "F.Cu") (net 38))
 (segment (start 103.019999 54.764001) (end 103.87 53.914) (width 0.4) (layer "F.Cu") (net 38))
 (segment (start 103.87 63.566) (end 103.019999 62.715999) (width 0.4) (layer "F.Cu") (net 38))
 (segment (start 103.019999 59.336001) (end 103.87 58.486) (width 0.4) (layer "F.Cu") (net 38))
 (segment (start 103.019999 62.715999) (end 103.019999 59.336001) (width 0.4) (layer "F.Cu") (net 38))
 (segment (start 103.87 68.646) (end 103.019999 67.795999) (width 0.4) (layer "F.Cu") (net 38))
 (segment (start 103.019999 67.795999) (end 103.019999 64.416001) (width 0.4) (layer "F.Cu") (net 38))
 (segment (start 103.019999 64.416001) (end 103.87 63.566) (width 0.4) (layer "F.Cu") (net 38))
 (segment (start 103.87 73.726) (end 102.720001 72.576001) (width 0.4) (layer "F.Cu") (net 38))
 (segment (start 102.720001 72.576001) (end 102.720001 69.795999) (width 0.4) (layer "F.Cu") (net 38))
 (segment (start 102.720001 69.795999) (end 103.87 68.646) (width 0.4) (layer "F.Cu") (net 38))
 (segment (start 103.87 78.806) (end 103.019999 77.955999) (width 0.4) (layer "F.Cu") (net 38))
 (segment (start 103.019999 77.955999) (end 103.019999 74.576001) (width 0.4) (layer "F.Cu") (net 38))
 (segment (start 103.019999 74.576001) (end 103.87 73.726) (width 0.4) (layer "F.Cu") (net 38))
 (segment (start 103.87 83.886) (end 103.019999 83.035999) (width 0.4) (layer "F.Cu") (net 38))
 (segment (start 103.019999 83.035999) (end 103.019999 79.656001) (width 0.4) (layer "F.Cu") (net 38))
 (segment (start 103.019999 79.656001) (end 103.87 78.806) (width 0.4) (layer "F.Cu") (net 38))
 (segment (start 103.87 88.966) (end 103.019999 88.115999) (width 0.4) (layer "F.Cu") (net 38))
 (segment (start 103.019999 88.115999) (end 103.019999 84.736001) (width 0.4) (layer "F.Cu") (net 38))
 (segment (start 103.019999 84.736001) (end 103.87 83.886) (width 0.4) (layer "F.Cu") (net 38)))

